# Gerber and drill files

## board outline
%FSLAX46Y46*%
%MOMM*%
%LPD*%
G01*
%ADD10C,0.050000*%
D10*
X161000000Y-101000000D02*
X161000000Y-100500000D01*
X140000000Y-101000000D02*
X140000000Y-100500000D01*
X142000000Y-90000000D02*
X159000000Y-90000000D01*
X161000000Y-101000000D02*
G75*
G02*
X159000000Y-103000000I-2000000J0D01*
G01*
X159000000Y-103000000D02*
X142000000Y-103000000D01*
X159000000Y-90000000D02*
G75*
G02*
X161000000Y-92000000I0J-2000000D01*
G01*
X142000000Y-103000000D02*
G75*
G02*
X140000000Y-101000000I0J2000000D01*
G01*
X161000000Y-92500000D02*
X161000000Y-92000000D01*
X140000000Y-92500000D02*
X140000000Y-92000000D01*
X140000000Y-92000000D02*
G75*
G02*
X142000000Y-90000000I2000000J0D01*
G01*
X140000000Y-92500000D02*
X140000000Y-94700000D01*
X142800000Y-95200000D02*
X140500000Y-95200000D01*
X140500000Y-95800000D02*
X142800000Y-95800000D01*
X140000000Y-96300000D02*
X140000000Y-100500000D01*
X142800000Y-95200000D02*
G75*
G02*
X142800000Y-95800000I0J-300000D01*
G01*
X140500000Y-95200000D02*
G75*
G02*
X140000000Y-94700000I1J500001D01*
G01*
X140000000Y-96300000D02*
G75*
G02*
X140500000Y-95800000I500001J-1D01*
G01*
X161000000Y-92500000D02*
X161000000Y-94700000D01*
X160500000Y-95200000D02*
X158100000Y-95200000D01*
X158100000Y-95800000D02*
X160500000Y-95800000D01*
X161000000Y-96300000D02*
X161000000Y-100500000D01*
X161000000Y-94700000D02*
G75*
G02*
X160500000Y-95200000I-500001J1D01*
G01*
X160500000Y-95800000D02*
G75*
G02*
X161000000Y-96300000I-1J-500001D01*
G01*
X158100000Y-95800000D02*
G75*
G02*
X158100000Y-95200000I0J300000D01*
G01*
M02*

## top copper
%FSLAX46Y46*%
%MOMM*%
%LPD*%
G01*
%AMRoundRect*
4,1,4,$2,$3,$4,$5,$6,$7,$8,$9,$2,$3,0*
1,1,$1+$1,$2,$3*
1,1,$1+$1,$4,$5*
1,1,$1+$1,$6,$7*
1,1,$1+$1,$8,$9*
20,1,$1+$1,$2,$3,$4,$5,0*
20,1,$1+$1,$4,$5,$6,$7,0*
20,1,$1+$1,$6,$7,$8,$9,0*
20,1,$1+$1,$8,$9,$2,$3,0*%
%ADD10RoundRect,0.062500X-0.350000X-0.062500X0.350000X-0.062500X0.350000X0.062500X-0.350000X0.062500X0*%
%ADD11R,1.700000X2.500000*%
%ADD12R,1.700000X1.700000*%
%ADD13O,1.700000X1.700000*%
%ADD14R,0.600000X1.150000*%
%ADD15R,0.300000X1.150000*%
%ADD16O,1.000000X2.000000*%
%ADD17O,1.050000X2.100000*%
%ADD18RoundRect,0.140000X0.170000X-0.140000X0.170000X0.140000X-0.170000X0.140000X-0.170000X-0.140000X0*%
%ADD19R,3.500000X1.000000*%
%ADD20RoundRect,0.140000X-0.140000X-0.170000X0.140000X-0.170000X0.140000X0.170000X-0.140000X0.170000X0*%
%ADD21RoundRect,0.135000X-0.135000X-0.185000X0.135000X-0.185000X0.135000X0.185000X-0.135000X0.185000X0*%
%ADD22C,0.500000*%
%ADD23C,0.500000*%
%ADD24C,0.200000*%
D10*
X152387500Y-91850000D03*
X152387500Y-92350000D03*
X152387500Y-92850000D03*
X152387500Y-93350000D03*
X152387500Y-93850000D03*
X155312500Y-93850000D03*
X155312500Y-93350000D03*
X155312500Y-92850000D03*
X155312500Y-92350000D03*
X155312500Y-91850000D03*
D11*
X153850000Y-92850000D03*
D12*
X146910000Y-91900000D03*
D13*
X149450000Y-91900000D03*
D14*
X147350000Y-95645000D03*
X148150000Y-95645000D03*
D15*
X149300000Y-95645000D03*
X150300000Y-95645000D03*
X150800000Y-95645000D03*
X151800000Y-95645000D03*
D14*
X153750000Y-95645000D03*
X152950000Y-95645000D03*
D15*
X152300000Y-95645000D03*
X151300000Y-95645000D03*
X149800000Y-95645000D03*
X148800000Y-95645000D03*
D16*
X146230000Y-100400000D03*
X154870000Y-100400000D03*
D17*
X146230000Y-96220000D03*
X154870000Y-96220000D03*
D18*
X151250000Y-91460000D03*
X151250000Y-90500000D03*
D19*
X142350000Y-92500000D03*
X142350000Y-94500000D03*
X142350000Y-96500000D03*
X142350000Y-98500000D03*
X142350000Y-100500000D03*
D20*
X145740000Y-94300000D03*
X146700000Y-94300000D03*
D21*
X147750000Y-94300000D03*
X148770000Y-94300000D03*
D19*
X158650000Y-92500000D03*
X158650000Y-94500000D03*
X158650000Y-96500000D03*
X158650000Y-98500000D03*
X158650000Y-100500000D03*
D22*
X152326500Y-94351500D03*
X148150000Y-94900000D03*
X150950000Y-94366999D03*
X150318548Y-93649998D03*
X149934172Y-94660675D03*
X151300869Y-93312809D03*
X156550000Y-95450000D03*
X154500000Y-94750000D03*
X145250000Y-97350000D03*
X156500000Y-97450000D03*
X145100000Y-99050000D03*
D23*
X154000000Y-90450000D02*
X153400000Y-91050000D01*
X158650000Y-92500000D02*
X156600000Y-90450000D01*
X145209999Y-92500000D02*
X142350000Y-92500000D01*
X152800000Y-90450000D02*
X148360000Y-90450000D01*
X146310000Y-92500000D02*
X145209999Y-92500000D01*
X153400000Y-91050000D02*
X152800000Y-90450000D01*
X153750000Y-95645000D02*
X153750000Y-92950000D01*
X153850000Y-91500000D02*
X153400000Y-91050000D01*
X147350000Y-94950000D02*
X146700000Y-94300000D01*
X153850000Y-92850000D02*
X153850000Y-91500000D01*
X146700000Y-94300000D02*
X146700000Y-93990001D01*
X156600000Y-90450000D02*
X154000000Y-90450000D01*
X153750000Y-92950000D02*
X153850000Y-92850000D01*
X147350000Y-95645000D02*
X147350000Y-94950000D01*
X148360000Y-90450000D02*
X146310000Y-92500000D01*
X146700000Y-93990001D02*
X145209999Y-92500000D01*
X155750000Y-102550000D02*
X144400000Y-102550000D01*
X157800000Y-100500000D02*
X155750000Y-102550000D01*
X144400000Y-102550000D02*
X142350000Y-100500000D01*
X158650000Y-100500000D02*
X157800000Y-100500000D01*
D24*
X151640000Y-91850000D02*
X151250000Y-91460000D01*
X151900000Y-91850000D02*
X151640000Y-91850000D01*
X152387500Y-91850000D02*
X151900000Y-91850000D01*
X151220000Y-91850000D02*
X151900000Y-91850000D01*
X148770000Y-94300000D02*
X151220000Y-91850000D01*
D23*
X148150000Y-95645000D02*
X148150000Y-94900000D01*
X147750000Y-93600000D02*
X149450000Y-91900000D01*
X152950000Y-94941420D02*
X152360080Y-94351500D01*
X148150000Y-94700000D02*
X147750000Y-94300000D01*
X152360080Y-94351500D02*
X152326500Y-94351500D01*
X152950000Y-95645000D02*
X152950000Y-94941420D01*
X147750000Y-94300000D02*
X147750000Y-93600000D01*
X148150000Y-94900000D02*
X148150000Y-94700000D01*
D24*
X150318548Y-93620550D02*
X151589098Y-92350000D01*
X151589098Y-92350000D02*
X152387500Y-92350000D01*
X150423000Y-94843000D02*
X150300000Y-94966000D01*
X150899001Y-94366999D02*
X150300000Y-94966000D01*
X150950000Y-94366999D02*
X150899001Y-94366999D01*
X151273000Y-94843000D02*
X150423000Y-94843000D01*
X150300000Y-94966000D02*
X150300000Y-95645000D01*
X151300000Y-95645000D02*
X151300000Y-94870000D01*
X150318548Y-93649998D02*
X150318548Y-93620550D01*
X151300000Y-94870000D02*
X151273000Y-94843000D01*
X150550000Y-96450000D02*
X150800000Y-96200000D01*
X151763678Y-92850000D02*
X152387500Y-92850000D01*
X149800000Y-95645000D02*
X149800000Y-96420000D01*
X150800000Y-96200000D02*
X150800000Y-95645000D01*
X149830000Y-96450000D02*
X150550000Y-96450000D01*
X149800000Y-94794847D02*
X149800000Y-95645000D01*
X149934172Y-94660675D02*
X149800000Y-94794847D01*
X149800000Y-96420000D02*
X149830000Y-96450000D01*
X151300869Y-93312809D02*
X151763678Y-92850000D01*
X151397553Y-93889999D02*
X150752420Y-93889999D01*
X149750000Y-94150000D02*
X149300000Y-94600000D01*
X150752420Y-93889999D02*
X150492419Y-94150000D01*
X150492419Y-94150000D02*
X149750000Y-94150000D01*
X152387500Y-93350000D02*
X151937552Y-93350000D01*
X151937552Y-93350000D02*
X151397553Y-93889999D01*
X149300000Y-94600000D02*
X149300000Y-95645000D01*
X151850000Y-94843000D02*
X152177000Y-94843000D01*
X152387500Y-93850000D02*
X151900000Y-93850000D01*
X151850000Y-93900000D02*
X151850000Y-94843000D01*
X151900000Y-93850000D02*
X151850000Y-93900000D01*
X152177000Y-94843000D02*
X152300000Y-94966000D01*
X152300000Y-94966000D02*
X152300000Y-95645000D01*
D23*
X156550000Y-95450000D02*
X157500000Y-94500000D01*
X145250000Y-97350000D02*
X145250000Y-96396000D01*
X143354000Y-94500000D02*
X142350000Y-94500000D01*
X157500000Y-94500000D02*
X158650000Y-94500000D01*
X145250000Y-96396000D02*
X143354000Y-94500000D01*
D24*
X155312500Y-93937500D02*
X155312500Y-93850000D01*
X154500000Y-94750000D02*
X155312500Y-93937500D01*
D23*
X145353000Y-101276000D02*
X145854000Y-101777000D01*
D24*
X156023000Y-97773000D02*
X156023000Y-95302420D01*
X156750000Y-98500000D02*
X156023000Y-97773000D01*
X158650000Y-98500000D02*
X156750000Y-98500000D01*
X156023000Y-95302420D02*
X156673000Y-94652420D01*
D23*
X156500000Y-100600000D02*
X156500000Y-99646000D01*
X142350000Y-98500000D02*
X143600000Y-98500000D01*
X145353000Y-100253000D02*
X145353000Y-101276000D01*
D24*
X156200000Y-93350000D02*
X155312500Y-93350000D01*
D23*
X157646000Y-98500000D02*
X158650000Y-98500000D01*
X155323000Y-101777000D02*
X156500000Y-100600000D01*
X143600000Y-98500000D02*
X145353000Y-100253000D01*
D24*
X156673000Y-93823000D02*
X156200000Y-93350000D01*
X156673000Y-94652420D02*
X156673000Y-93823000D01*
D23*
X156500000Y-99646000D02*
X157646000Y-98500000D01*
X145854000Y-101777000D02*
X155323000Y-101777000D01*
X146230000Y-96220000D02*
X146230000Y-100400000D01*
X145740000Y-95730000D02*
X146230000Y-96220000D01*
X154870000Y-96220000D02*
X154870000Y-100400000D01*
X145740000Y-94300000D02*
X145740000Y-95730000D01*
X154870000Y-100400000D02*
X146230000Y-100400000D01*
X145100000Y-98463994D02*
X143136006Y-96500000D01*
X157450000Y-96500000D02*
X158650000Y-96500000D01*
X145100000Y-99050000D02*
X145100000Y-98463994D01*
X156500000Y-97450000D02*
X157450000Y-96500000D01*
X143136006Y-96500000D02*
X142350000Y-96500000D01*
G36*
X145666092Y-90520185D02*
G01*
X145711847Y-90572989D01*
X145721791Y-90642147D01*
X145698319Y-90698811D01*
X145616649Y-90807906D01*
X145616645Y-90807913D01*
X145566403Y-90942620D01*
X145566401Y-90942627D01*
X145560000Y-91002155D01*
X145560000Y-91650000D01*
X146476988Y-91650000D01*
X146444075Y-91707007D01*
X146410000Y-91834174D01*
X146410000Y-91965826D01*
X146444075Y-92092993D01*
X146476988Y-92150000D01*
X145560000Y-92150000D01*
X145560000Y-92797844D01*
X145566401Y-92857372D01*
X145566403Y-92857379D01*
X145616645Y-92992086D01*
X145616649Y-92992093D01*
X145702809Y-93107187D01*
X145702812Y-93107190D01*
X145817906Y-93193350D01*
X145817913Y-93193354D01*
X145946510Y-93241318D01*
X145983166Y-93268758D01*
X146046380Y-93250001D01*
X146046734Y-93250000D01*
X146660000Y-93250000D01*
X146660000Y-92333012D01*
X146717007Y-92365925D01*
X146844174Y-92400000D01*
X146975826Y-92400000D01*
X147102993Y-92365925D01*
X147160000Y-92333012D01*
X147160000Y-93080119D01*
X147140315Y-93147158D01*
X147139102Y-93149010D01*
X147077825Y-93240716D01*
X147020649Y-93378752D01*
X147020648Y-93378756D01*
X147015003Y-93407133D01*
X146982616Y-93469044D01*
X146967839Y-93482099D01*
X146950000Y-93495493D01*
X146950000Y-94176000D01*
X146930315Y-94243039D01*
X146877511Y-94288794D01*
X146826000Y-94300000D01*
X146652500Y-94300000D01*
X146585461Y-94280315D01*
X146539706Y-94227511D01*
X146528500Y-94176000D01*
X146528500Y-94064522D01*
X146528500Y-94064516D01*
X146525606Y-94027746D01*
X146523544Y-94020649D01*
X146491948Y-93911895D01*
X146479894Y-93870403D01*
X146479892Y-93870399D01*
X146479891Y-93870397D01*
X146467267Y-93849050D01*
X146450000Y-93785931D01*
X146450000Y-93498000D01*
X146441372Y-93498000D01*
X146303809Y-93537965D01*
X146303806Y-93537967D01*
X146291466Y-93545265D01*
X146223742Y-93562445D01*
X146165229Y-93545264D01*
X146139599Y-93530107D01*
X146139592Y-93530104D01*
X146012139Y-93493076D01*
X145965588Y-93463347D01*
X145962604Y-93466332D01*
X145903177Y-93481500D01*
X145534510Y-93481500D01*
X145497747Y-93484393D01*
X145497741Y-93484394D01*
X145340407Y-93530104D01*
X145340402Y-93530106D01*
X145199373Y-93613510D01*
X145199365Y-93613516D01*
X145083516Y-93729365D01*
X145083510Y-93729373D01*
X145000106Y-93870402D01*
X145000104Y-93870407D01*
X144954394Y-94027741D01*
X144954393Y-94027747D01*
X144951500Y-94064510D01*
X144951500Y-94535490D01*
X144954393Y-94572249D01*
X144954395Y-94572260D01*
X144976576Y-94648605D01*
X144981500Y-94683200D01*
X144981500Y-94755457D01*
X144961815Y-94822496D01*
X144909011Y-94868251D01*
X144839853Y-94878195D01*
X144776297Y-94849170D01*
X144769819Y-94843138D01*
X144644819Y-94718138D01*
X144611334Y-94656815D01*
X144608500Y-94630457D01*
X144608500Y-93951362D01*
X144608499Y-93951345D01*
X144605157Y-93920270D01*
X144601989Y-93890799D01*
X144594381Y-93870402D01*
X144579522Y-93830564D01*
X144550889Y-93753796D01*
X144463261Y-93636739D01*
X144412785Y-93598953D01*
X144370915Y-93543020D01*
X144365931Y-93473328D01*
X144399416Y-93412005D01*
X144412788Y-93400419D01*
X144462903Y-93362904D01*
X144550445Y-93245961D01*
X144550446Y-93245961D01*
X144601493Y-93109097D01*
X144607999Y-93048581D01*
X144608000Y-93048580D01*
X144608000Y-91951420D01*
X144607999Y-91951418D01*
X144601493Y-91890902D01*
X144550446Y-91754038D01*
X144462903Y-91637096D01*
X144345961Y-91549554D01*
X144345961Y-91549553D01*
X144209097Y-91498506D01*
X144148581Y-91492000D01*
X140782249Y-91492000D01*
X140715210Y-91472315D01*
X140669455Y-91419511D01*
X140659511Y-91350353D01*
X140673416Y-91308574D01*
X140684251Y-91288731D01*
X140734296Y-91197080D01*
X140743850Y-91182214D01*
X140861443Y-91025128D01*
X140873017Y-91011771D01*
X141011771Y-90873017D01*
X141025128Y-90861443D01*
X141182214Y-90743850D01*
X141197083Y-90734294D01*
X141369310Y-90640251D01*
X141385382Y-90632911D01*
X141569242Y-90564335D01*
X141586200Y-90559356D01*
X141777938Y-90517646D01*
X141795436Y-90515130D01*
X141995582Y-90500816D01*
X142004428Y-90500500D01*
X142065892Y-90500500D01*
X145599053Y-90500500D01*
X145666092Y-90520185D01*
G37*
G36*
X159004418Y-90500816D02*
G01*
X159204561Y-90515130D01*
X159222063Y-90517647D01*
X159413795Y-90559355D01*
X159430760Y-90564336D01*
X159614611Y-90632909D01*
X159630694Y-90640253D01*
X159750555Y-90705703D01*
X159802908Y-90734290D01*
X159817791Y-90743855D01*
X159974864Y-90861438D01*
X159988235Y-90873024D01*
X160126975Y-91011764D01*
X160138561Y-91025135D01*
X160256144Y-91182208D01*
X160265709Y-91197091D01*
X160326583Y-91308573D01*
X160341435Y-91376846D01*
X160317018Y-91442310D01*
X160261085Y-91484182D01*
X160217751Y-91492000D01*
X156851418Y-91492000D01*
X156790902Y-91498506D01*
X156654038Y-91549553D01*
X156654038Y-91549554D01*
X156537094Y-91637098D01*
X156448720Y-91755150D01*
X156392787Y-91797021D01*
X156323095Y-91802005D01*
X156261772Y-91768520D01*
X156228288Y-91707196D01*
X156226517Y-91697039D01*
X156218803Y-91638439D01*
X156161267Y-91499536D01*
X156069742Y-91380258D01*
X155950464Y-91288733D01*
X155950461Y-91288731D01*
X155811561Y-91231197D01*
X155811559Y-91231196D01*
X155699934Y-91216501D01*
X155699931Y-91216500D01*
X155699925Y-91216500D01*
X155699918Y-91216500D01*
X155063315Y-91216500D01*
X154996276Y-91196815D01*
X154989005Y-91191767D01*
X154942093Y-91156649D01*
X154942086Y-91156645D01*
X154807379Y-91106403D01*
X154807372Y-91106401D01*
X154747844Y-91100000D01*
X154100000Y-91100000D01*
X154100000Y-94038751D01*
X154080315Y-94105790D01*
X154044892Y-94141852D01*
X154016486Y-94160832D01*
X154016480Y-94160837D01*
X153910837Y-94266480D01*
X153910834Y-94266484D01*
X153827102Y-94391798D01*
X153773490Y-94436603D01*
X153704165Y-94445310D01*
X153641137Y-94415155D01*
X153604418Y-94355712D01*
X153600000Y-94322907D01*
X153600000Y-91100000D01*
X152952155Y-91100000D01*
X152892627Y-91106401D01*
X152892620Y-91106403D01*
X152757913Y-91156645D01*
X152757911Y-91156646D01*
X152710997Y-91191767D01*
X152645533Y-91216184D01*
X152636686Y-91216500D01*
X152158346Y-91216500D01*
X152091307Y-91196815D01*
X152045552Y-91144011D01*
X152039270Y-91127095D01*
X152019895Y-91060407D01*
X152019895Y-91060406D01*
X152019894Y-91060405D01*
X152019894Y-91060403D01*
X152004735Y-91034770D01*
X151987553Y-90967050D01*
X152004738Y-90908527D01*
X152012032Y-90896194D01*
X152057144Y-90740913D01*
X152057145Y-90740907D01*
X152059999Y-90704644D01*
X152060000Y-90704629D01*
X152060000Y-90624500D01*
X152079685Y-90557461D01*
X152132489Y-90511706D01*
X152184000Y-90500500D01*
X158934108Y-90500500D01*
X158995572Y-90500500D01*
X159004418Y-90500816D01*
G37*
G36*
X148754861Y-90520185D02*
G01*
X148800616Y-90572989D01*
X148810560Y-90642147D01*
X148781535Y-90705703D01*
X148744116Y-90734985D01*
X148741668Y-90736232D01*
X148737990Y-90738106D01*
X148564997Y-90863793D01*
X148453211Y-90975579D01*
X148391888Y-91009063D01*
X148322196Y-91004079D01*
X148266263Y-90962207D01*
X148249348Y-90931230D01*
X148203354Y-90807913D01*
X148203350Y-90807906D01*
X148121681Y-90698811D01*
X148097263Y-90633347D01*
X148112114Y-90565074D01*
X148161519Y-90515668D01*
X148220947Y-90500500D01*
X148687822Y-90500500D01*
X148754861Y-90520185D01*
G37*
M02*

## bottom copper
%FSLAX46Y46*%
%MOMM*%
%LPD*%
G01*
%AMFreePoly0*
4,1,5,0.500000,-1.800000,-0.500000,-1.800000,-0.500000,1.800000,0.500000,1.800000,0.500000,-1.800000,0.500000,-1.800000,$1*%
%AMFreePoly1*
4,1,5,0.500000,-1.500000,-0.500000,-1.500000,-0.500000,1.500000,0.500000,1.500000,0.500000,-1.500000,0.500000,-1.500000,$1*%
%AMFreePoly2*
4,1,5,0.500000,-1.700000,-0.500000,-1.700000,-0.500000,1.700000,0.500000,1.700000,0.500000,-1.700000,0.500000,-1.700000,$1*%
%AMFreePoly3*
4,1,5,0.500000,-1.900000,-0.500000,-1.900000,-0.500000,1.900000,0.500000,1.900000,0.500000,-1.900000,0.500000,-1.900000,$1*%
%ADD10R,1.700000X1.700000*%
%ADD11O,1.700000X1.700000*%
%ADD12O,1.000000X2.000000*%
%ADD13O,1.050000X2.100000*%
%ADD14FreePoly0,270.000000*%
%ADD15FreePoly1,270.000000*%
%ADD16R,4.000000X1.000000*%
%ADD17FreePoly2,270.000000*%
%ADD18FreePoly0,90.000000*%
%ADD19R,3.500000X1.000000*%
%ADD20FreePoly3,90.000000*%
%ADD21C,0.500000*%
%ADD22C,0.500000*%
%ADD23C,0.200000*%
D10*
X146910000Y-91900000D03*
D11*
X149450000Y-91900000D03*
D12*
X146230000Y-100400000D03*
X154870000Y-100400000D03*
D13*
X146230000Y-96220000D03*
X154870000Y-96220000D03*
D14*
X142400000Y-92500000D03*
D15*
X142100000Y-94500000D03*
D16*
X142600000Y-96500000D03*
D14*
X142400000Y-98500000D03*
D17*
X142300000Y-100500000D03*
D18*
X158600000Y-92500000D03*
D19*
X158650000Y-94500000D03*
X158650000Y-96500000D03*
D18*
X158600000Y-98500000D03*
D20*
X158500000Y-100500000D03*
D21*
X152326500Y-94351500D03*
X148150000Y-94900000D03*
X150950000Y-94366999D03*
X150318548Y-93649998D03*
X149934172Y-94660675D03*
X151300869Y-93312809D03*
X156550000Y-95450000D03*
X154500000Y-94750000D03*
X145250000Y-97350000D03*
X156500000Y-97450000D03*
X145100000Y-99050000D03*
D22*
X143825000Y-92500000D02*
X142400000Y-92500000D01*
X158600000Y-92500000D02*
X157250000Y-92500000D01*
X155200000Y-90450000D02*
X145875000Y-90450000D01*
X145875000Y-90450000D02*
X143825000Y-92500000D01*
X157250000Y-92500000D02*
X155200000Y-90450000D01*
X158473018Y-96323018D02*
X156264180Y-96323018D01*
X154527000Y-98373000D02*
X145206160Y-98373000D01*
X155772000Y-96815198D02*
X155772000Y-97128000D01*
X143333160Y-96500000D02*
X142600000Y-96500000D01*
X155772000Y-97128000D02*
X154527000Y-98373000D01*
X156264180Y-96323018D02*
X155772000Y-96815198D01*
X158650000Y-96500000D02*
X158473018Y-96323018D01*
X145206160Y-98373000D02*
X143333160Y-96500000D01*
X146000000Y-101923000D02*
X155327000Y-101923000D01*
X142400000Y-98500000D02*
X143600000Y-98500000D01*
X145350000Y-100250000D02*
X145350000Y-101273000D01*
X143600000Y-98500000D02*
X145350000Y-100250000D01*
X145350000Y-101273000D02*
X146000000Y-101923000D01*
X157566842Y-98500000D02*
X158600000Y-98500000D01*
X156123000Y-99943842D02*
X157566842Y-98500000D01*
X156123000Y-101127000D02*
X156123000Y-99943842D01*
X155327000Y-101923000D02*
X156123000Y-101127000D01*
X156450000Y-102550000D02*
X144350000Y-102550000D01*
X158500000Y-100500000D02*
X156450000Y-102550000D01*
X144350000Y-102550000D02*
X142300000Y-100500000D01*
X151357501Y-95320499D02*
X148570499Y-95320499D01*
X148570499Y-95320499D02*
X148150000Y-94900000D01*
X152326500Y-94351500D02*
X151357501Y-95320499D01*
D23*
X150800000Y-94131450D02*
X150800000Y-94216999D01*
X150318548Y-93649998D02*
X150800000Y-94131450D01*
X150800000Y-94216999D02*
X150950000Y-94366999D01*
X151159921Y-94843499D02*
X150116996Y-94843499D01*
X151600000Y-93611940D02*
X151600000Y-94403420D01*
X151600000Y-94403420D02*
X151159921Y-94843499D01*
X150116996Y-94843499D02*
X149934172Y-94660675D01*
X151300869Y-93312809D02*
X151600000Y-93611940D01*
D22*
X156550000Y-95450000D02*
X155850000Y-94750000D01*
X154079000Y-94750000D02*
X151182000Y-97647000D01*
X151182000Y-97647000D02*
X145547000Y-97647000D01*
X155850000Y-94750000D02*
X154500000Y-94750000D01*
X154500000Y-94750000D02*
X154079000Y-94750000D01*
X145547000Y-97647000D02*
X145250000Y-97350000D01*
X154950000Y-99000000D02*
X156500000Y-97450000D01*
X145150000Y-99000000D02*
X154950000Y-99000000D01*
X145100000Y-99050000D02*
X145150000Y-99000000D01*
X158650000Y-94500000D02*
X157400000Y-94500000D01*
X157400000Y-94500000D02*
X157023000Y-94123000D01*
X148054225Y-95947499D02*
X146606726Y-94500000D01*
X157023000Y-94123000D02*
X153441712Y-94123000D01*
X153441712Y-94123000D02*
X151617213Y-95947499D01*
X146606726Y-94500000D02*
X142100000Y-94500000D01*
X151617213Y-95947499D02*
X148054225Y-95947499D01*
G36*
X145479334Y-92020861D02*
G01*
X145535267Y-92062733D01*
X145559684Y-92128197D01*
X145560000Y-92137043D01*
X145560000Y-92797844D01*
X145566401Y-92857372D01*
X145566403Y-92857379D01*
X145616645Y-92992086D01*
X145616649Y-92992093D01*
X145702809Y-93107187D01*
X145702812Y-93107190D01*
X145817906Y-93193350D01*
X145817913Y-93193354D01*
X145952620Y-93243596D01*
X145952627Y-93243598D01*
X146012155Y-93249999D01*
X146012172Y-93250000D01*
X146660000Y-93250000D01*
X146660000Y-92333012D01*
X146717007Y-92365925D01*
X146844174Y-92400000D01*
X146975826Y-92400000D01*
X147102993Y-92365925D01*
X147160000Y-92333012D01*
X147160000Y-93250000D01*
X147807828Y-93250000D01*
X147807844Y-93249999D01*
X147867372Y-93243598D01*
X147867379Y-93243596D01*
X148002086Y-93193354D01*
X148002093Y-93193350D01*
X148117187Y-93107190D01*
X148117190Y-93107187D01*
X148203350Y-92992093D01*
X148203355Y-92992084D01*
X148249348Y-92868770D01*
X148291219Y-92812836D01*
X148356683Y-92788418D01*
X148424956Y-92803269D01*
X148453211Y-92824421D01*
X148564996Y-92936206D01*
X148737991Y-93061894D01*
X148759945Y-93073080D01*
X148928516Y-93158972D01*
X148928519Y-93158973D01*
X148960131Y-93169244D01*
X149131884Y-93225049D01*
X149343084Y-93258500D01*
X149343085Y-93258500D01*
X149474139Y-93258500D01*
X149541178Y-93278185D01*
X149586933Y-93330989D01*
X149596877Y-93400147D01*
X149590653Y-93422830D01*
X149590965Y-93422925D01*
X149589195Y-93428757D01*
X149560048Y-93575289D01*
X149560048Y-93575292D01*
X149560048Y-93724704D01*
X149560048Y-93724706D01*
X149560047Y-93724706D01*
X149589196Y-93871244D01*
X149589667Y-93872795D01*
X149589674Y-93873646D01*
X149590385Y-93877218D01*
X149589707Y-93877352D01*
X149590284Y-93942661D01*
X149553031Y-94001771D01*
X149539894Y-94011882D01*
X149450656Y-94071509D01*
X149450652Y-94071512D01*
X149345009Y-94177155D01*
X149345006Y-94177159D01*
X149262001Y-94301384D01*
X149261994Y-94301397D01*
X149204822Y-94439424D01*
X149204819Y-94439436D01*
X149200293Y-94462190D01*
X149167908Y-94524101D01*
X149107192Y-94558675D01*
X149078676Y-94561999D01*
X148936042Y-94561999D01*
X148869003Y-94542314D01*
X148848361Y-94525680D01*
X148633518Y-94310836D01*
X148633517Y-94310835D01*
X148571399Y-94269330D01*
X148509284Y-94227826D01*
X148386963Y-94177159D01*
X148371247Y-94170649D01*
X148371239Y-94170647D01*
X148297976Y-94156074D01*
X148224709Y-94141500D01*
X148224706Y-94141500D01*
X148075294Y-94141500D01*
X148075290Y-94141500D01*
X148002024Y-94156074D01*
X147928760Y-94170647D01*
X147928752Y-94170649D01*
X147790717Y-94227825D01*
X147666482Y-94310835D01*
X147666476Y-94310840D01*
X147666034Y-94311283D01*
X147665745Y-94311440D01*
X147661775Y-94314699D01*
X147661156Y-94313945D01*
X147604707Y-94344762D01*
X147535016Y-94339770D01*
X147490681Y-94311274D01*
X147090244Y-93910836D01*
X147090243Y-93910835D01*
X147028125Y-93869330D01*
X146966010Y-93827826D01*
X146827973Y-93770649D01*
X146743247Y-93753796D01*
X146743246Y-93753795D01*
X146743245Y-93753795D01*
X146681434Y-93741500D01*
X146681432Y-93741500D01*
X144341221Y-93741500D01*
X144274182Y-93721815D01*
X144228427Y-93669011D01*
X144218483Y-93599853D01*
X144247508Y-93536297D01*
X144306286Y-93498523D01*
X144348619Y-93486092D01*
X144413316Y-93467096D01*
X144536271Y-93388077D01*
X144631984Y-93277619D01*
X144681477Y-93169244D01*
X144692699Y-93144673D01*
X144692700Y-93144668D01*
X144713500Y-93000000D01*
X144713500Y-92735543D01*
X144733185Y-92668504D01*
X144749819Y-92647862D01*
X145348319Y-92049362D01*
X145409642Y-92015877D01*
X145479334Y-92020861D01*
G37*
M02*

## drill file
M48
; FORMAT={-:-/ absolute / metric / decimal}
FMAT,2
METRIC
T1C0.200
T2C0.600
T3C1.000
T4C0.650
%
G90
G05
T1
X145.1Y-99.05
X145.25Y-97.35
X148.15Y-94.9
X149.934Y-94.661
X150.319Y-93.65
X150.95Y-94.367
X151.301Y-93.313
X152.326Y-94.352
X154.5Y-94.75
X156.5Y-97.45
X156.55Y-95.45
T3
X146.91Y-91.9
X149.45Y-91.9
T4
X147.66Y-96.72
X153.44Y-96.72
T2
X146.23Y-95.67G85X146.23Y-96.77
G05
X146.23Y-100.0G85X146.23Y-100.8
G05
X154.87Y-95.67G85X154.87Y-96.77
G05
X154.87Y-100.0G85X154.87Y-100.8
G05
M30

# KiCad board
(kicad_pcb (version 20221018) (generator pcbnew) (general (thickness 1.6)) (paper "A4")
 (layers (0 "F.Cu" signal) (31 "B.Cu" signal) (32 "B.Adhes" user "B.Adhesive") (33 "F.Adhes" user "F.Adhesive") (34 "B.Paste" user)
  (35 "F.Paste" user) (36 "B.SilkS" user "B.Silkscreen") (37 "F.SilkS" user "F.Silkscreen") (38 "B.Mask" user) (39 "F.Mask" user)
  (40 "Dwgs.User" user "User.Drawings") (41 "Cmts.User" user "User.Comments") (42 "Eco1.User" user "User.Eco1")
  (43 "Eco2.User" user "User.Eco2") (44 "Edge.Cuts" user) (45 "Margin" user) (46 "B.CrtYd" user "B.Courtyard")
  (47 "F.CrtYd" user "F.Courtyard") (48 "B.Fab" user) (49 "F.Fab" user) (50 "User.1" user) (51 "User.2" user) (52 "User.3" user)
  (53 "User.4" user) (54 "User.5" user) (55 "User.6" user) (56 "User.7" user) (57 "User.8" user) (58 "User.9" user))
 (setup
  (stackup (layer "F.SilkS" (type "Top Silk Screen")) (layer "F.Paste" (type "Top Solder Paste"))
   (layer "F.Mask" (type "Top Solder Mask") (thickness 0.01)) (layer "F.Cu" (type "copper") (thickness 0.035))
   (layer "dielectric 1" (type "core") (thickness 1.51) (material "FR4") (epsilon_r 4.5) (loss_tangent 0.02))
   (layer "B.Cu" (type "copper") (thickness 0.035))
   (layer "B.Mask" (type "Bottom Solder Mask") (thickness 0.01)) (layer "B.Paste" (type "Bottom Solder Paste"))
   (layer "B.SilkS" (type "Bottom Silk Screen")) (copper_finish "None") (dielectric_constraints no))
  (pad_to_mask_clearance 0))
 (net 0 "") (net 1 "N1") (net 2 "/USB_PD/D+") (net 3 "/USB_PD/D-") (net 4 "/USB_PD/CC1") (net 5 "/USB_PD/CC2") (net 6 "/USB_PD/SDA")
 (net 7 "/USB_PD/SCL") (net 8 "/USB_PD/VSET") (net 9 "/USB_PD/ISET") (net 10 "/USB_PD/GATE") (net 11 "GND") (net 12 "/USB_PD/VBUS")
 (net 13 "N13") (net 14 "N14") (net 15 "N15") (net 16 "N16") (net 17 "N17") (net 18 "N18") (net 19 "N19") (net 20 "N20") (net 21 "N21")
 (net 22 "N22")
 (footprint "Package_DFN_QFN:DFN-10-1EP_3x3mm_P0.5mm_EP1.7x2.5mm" (layer "F.Cu") (at 153.85 92.85)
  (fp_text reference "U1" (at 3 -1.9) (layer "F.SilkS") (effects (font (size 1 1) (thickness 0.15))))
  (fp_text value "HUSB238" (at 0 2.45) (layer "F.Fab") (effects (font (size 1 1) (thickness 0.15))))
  (pad "" smd roundrect (at -0.425 -0.625) (size 0.69 1.01) (layers "F.Paste") (roundrect_rratio 0.25))
  (pad "" smd roundrect (at -0.425 0.625) (size 0.69 1.01) (layers "F.Paste") (roundrect_rratio 0.25))
  (pad "" smd roundrect (at 0.425 -0.625) (size 0.69 1.01) (layers "F.Paste") (roundrect_rratio 0.25))
  (pad "" smd roundrect (at 0.425 0.625) (size 0.69 1.01) (layers "F.Paste") (roundrect_rratio 0.25))
  (pad "1" smd roundrect (at -1.4625 -1) (size 0.825 0.25) (layers "F.Cu" "F.Paste" "F.Mask") (roundrect_rratio 0.25) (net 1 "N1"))
  (pad "2" smd roundrect (at -1.4625 -0.5) (size 0.825 0.25) (layers "F.Cu" "F.Paste" "F.Mask") (roundrect_rratio 0.25) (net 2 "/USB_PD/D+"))
  (pad "3" smd roundrect (at -1.4625 0) (size 0.825 0.25) (layers "F.Cu" "F.Paste" "F.Mask") (roundrect_rratio 0.25) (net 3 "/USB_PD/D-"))
  (pad "4" smd roundrect (at -1.4625 0.5) (size 0.825 0.25) (layers "F.Cu" "F.Paste" "F.Mask") (roundrect_rratio 0.25) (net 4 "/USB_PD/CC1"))
  (pad "5" smd roundrect (at -1.4625 1) (size 0.825 0.25) (layers "F.Cu" "F.Paste" "F.Mask") (roundrect_rratio 0.25) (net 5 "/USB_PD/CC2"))
  (pad "6" smd roundrect (at 1.4625 1) (size 0.825 0.25) (layers "F.Cu" "F.Paste" "F.Mask") (roundrect_rratio 0.25) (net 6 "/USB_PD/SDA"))
  (pad "7" smd roundrect (at 1.4625 0.5) (size 0.825 0.25) (layers "F.Cu" "F.Paste" "F.Mask") (roundrect_rratio 0.25) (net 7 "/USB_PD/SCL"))
  (pad "8" smd roundrect (at 1.4625 0) (size 0.825 0.25) (layers "F.Cu" "F.Paste" "F.Mask") (roundrect_rratio 0.25) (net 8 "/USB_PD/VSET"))
  (pad "9" smd roundrect (at 1.4625 -0.5) (size 0.825 0.25) (layers "F.Cu" "F.Paste" "F.Mask") (roundrect_rratio 0.25)
   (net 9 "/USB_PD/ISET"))
  (pad "10" smd roundrect (at 1.4625 -1) (size 0.825 0.25) (layers "F.Cu" "F.Paste" "F.Mask") (roundrect_rratio 0.25)
   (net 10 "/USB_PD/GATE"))
  (pad "11" smd rect (at 0 0) (size 1.7 2.5) (layers "F.Cu" "F.Mask") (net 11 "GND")))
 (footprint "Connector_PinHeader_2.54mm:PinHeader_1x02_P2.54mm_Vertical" (layer "F.Cu") (at 146.91 91.9 90)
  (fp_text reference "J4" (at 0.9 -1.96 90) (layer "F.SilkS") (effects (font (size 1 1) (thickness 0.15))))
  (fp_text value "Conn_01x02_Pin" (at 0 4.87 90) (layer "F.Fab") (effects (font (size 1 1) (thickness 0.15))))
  (pad "1" thru_hole rect (at 0 0 90) (size 1.7 1.7) (drill 1) (layers "*.Cu" "*.Mask") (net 11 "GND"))
  (pad "2" thru_hole oval (at 0 2.54 90) (size 1.7 1.7) (drill 1) (layers "*.Cu" "*.Mask") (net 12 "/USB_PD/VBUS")))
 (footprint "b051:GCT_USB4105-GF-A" (layer "F.Cu") (at 150.55 100.4)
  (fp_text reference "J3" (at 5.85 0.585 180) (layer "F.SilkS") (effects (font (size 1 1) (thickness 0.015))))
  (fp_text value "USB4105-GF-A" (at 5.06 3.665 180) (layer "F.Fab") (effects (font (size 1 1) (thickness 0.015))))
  (pad "" np_thru_hole circle (at -2.89 -3.68) (size 0.65 0.65) (drill 0.65) (layers "*.Cu" "*.Mask"))
  (pad "" np_thru_hole circle (at 2.89 -3.68) (size 0.65 0.65) (drill 0.65) (layers "*.Cu" "*.Mask"))
  (pad "A1/B12" smd rect (at -3.2 -4.755) (size 0.6 1.15) (layers "F.Cu" "F.Paste" "F.Mask") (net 11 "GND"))
  (pad "A4/B9" smd rect (at -2.4 -4.755) (size 0.6 1.15) (layers "F.Cu" "F.Paste" "F.Mask") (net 12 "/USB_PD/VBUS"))
  (pad "A5" smd rect (at -1.25 -4.755) (size 0.3 1.15) (layers "F.Cu" "F.Paste" "F.Mask") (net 4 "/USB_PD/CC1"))
  (pad "A6" smd rect (at -0.25 -4.755) (size 0.3 1.15) (layers "F.Cu" "F.Paste" "F.Mask") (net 2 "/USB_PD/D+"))
  (pad "A7" smd rect (at 0.25 -4.755) (size 0.3 1.15) (layers "F.Cu" "F.Paste" "F.Mask") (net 3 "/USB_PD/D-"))
  (pad "A8" smd rect (at 1.25 -4.755) (size 0.3 1.15) (layers "F.Cu" "F.Paste" "F.Mask") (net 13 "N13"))
  (pad "B1/A12" smd rect (at 3.2 -4.755) (size 0.6 1.15) (layers "F.Cu" "F.Paste" "F.Mask") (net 11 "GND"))
  (pad "B4/A9" smd rect (at 2.4 -4.755) (size 0.6 1.15) (layers "F.Cu" "F.Paste" "F.Mask") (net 12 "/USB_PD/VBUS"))
  (pad "B5" smd rect (at 1.75 -4.755) (size 0.3 1.15) (layers "F.Cu" "F.Paste" "F.Mask") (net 5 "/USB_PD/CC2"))
  (pad "B6" smd rect (at 0.75 -4.755) (size 0.3 1.15) (layers "F.Cu" "F.Paste" "F.Mask") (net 2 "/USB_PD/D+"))
  (pad "B7" smd rect (at -0.75 -4.755) (size 0.3 1.15) (layers "F.Cu" "F.Paste" "F.Mask") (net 3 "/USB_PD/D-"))
  (pad "B8" smd rect (at -1.75 -4.755) (size 0.3 1.15) (layers "F.Cu" "F.Paste" "F.Mask") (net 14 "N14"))
  (pad "G1" thru_hole oval (at -4.32 0) (size 1 2) (drill oval 0.6 1.4) (layers "*.Cu" "*.Mask") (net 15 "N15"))
  (pad "G2" thru_hole oval (at 4.32 0) (size 1 2) (drill oval 0.6 1.4) (layers "*.Cu" "*.Mask") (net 15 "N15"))
  (pad "G3" thru_hole oval (at -4.32 -4.18) (size 1.05 2.1) (drill oval 0.6 1.7) (layers "*.Cu" "*.Mask") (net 15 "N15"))
  (pad "G4" thru_hole oval (at 4.32 -4.18) (size 1.05 2.1) (drill oval 0.6 1.7) (layers "*.Cu" "*.Mask") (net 15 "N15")))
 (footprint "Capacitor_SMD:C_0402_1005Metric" (layer "F.Cu") (at 151.25 90.98 90)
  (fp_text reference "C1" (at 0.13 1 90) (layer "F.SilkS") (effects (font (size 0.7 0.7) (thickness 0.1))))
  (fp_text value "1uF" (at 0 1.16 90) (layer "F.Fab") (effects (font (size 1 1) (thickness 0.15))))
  (pad "1" smd roundrect (at -0.48 0 90) (size 0.56 0.62) (layers "F.Cu" "F.Paste" "F.Mask") (roundrect_rratio 0.25) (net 1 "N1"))
  (pad "2" smd roundrect (at 0.48 0 90) (size 0.56 0.62) (layers "F.Cu" "F.Paste" "F.Mask") (roundrect_rratio 0.25) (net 11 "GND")))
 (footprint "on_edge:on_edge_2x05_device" (layer "F.Cu") (at 140 96.5 -90)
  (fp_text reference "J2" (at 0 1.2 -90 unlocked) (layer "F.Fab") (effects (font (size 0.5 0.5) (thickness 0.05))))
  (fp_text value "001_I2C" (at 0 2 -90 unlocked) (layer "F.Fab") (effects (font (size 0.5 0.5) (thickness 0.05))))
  (fp_line (start -4 0) (end -1.8 0) (stroke (width 0.05) (type solid)) (layer "Edge.Cuts"))
  (fp_line (start -1.3 -2.8) (end -1.3 -0.5) (stroke (width 0.05) (type solid)) (layer "Edge.Cuts"))
  (fp_line (start -0.7 -0.5) (end -0.7 -2.8) (stroke (width 0.05) (type solid)) (layer "Edge.Cuts"))
  (fp_line (start -0.2 0) (end 4 0) (stroke (width 0.05) (type solid)) (layer "Edge.Cuts"))
  (fp_arc (start -1.3 -2.8) (mid -1 -3.1) (end -0.7 -2.8) (stroke (width 0.05) (type solid)) (layer "Edge.Cuts"))
  (fp_arc (start -1.3 -0.5) (mid -1.446447 -0.146447) (end -1.8 0) (stroke (width 0.05) (type solid)) (layer "Edge.Cuts"))
  (fp_arc (start -0.2 0) (mid -0.553553 -0.146447) (end -0.7 -0.5) (stroke (width 0.05) (type solid)) (layer "Edge.Cuts"))
  (pad "1" smd rect (at -4 -2.35 90) (size 1 3.5) (layers "F.Cu" "F.Mask") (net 11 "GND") (zone_connect 0))
  (pad "2" smd rect (at -2 -2.35 270) (size 1 3.5) (layers "F.Cu" "F.Mask") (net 6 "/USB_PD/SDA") (zone_connect 0))
  (pad "3" smd rect (at 0 -2.35 270) (size 1 3.5) (layers "F.Cu" "F.Mask") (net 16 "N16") (zone_connect 0))
  (pad "4" smd rect (at 2 -2.35 90) (size 1 3.5) (layers "F.Cu" "F.Mask") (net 7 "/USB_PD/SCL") (zone_connect 0))
  (pad "5" smd rect (at 4 -2.35 90) (size 1 3.5) (layers "F.Cu" "F.Mask") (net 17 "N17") (zone_connect 0))
  (pad "6" smd custom (at -4 -2.4 270) (size 1 3.6) (layers "B.Cu" "B.Mask") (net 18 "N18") (zone_connect 0)
   (options (clearance outline) (anchor rect)) (primitives))
  (pad "7" smd custom (at -2 -2.1 270) (size 1 3) (layers "B.Cu" "B.Mask") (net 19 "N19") (zone_connect 0)
   (options (clearance outline) (anchor rect)) (primitives))
  (pad "8" smd rect (at 0 -2.6 270) (size 1 4) (layers "B.Cu" "B.Mask") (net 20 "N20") (zone_connect 0))
  (pad "9" smd custom (at 2 -2.4 270) (size 1 3.6) (layers "B.Cu" "B.Mask") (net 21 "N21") (zone_connect 0)
   (options (clearance outline) (anchor rect)) (primitives))
  (pad "10" smd custom (at 4 -2.3 270) (size 1 3.4) (layers "B.Cu" "B.Mask") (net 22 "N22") (zone_connect 0)
   (options (clearance outline) (anchor rect)) (primitives))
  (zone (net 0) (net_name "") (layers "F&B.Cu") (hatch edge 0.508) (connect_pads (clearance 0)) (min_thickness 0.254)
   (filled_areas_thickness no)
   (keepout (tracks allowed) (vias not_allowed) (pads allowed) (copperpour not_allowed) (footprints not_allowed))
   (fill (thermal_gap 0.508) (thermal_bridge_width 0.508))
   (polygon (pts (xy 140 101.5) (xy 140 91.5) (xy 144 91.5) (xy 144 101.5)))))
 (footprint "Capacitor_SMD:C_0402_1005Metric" (layer "F.Cu") (at 146.22 94.3)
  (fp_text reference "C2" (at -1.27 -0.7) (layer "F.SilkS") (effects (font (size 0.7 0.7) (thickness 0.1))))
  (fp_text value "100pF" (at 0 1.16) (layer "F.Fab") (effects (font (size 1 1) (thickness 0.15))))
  (pad "1" smd roundrect (at -0.48 0) (size 0.56 0.62) (layers "F.Cu" "F.Paste" "F.Mask") (roundrect_rratio 0.25) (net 15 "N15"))
  (pad "2" smd roundrect (at 0.48 0) (size 0.56 0.62) (layers "F.Cu" "F.Paste" "F.Mask") (roundrect_rratio 0.25) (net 11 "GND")))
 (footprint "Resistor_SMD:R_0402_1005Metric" (layer "F.Cu") (at 148.26 94.3)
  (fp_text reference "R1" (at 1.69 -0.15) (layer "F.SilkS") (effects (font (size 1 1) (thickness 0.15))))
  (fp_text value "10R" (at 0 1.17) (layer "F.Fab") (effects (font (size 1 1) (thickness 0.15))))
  (pad "1" smd roundrect (at -0.51 0) (size 0.54 0.64) (layers "F.Cu" "F.Paste" "F.Mask") (roundrect_rratio 0.25) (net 12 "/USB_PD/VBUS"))
  (pad "2" smd roundrect (at 0.51 0) (size 0.54 0.64) (layers "F.Cu" "F.Paste" "F.Mask") (roundrect_rratio 0.25) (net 1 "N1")))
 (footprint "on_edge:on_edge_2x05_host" (layer "F.Cu") (at 161 96.5 -90)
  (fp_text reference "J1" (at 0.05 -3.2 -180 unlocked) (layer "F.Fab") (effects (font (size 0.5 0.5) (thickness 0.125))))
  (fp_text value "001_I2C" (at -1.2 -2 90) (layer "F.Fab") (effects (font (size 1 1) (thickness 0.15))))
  (fp_line (start -4 0) (end -1.8 0) (stroke (width 0.05) (type solid)) (layer "Edge.Cuts"))
  (fp_line (start -1.3 0.5) (end -1.3 2.9) (stroke (width 0.05) (type solid)) (layer "Edge.Cuts"))
  (fp_line (start -0.7 2.9) (end -0.7 0.5) (stroke (width 0.05) (type solid)) (layer "Edge.Cuts"))
  (fp_line (start -0.2 0) (end 4 0) (stroke (width 0.05) (type solid)) (layer "Edge.Cuts"))
  (fp_arc (start -1.8 0) (mid -1.446447 0.146447) (end -1.3 0.5) (stroke (width 0.05) (type solid)) (layer "Edge.Cuts"))
  (fp_arc (start -0.7 0.5) (mid -0.553553 0.146447) (end -0.2 0) (stroke (width 0.05) (type solid)) (layer "Edge.Cuts"))
  (fp_arc (start -0.7 2.9) (mid -1 3.2) (end -1.3 2.9) (stroke (width 0.05) (type solid)) (layer "Edge.Cuts"))
  (pad "1" smd rect (at -4 2.35 270) (size 1 3.5) (layers "F.Cu" "F.Mask") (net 11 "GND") (zone_connect 0))
  (pad "2" smd rect (at -2 2.35 270) (size 1 3.5) (layers "F.Cu" "F.Mask") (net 6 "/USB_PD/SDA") (zone_connect 0))
  (pad "3" smd rect (at 0 2.35 270) (size 1 3.5) (layers "F.Cu" "F.Mask") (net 16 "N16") (zone_connect 0))
  (pad "4" smd rect (at 2 2.35 270) (size 1 3.5) (layers "F.Cu" "F.Mask") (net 7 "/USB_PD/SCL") (zone_connect 0))
  (pad "5" smd rect (at 4 2.35 270) (size 1 3.5) (layers "F.Cu" "F.Mask") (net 17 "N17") (zone_connect 0))
  (pad "6" smd custom (at -4 2.4 90) (size 1 3.6) (layers "B.Cu" "B.Mask") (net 18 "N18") (zone_connect 0)
   (options (clearance outline) (anchor rect)) (primitives))
  (pad "7" smd rect (at -2 2.35 90) (size 1 3.5) (layers "B.Cu" "B.Mask") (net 19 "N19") (zone_connect 0))
  (pad "8" smd rect (at 0 2.35 90) (size 1 3.5) (layers "B.Cu" "B.Mask") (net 20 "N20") (zone_connect 0))
  (pad "9" smd custom (at 2 2.4 90) (size 1 3.6) (layers "B.Cu" "B.Mask") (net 21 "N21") (zone_connect 0)
   (options (clearance outline) (anchor rect)) (primitives))
  (pad "10" smd custom (at 4 2.5 90) (size 1 3.8) (layers "B.Cu" "B.Mask") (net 22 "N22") (zone_connect 0)
   (options (clearance outline) (anchor rect)) (primitives))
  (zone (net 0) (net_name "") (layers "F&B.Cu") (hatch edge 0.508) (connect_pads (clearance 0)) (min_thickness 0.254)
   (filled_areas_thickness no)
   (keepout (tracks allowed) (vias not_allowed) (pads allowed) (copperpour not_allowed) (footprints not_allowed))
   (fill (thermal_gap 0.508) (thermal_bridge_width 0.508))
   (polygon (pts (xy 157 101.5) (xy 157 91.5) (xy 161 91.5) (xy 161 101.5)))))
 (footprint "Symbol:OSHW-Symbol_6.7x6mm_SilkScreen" (layer "B.Cu") (at 150.6 97.6 180)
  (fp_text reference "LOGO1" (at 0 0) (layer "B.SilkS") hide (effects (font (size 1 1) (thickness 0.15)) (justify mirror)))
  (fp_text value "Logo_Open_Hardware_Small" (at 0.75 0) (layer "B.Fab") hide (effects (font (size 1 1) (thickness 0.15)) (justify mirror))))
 (gr_line (start 161 101) (end 161 100.5) (stroke (width 0.05) (type solid)) (layer "Edge.Cuts"))
 (gr_line (start 140 101) (end 140 100.5) (stroke (width 0.05) (type solid)) (layer "Edge.Cuts"))
 (gr_line (start 142 90) (end 159 90) (stroke (width 0.05) (type solid)) (layer "Edge.Cuts"))
 (gr_arc (start 161 101) (mid 160.414214 102.414214) (end 159 103) (stroke (width 0.05) (type solid)) (layer "Edge.Cuts"))
 (gr_line (start 159 103) (end 142 103) (stroke (width 0.05) (type solid)) (layer "Edge.Cuts"))
 (gr_arc (start 159 90) (mid 160.414214 90.585786) (end 161 92) (stroke (width 0.05) (type solid)) (layer "Edge.Cuts"))
 (gr_arc (start 142 103) (mid 140.585786 102.414214) (end 140 101) (stroke (width 0.05) (type solid)) (layer "Edge.Cuts"))
 (gr_line (start 161 92.5) (end 161 92) (stroke (width 0.05) (type solid)) (layer "Edge.Cuts"))
 (gr_line (start 140 92.5) (end 140 92) (stroke (width 0.05) (type solid)) (layer "Edge.Cuts"))
 (gr_arc (start 140 92) (mid 140.585786 90.585786) (end 142 90) (stroke (width 0.05) (type solid)) (layer "Edge.Cuts"))
 (segment (start 154 90.45) (end 153.4 91.05) (width 0.5) (layer "F.Cu") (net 11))
 (segment (start 158.65 92.5) (end 156.6 90.45) (width 0.5) (layer "F.Cu") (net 11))
 (segment (start 145.209999 92.5) (end 142.35 92.5) (width 0.5) (layer "F.Cu") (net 11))
 (segment (start 152.8 90.45) (end 148.36 90.45) (width 0.5) (layer "F.Cu") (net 11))
 (segment (start 146.31 92.5) (end 145.209999 92.5) (width 0.5) (layer "F.Cu") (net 11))
 (segment (start 153.4 91.05) (end 152.8 90.45) (width 0.5) (layer "F.Cu") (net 11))
 (segment (start 153.75 95.645) (end 153.75 92.95) (width 0.5) (layer "F.Cu") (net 11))
 (segment (start 153.85 91.5) (end 153.4 91.05) (width 0.5) (layer "F.Cu") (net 11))
 (segment (start 147.35 94.95) (end 146.7 94.3) (width 0.5) (layer "F.Cu") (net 11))
 (segment (start 153.85 92.85) (end 153.85 91.5) (width 0.5) (layer "F.Cu") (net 11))
 (segment (start 146.7 94.3) (end 146.7 93.990001) (width 0.5) (layer "F.Cu") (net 11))
 (segment (start 156.6 90.45) (end 154 90.45) (width 0.5) (layer "F.Cu") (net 11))
 (segment (start 153.75 92.95) (end 153.85 92.85) (width 0.5) (layer "F.Cu") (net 11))
 (segment (start 147.35 95.645) (end 147.35 94.95) (width 0.5) (layer "F.Cu") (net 11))
 (segment (start 148.36 90.45) (end 146.31 92.5) (width 0.5) (layer "F.Cu") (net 11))
 (segment (start 146.7 93.990001) (end 145.209999 92.5) (width 0.5) (layer "F.Cu") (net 11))
 (segment (start 143.825 92.5) (end 142.4 92.5) (width 0.5) (layer "B.Cu") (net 18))
 (segment (start 158.6 92.5) (end 157.25 92.5) (width 0.5) (layer "B.Cu") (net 18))
 (segment (start 155.2 90.45) (end 145.875 90.45) (width 0.5) (layer "B.Cu") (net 18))
 (segment (start 145.875 90.45) (end 143.825 92.5) (width 0.5) (layer "B.Cu") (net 18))
 (segment (start 157.25 92.5) (end 155.2 90.45) (width 0.5) (layer "B.Cu") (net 18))
 (segment (start 155.75 102.55) (end 144.4 102.55) (width 0.5) (layer "F.Cu") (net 17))
 (segment (start 157.8 100.5) (end 155.75 102.55) (width 0.5) (layer "F.Cu") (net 17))
 (segment (start 144.4 102.55) (end 142.35 100.5) (width 0.5) (layer "F.Cu") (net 17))
 (segment (start 158.65 100.5) (end 157.8 100.5) (width 0.5) (layer "F.Cu") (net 17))
 (segment (start 158.473018 96.323018) (end 156.26418 96.323018) (width 0.5) (layer "B.Cu") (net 20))
 (segment (start 154.527 98.373) (end 145.20616 98.373) (width 0.5) (layer "B.Cu") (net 20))
 (segment (start 155.772 96.815198) (end 155.772 97.128) (width 0.5) (layer "B.Cu") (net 20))
 (segment (start 143.33316 96.5) (end 142.6 96.5) (width 0.5) (layer "B.Cu") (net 20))
 (segment (start 155.772 97.128) (end 154.527 98.373) (width 0.5) (layer "B.Cu") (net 20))
 (segment (start 156.26418 96.323018) (end 155.772 96.815198) (width 0.5) (layer "B.Cu") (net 20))
 (segment (start 158.65 96.5) (end 158.473018 96.323018) (width 0.5) (layer "B.Cu") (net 20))
 (segment (start 145.20616 98.373) (end 143.33316 96.5) (width 0.5) (layer "B.Cu") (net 20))
 (segment (start 146 101.923) (end 155.327 101.923) (width 0.5) (layer "B.Cu") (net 21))
 (segment (start 142.4 98.5) (end 143.6 98.5) (width 0.5) (layer "B.Cu") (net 21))
 (segment (start 145.35 100.25) (end 145.35 101.273) (width 0.5) (layer "B.Cu") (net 21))
 (segment (start 143.6 98.5) (end 145.35 100.25) (width 0.5) (layer "B.Cu") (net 21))
 (segment (start 145.35 101.273) (end 146 101.923) (width 0.5) (layer "B.Cu") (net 21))
 (segment (start 157.566842 98.5) (end 158.6 98.5) (width 0.5) (layer "B.Cu") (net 21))
 (segment (start 156.123 99.943842) (end 157.566842 98.5) (width 0.5) (layer "B.Cu") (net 21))
 (segment (start 156.123 101.127) (end 156.123 99.943842) (width 0.5) (layer "B.Cu") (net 21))
 (segment (start 155.327 101.923) (end 156.123 101.127) (width 0.5) (layer "B.Cu") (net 21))
 (segment (start 156.45 102.55) (end 144.35 102.55) (width 0.5) (layer "B.Cu") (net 22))
 (segment (start 158.5 100.5) (end 156.45 102.55) (width 0.5) (layer "B.Cu") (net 22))
 (segment (start 144.35 102.55) (end 142.3 100.5) (width 0.5) (layer "B.Cu") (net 22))
 (segment (start 151.64 91.85) (end 151.25 91.46) (width 0.2) (layer "F.Cu") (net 1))
 (segment (start 151.9 91.85) (end 151.64 91.85) (width 0.2) (layer "F.Cu") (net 1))
 (segment (start 152.3875 91.85) (end 151.9 91.85) (width 0.2) (layer "F.Cu") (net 1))
 (segment (start 151.22 91.85) (end 151.9 91.85) (width 0.2) (layer "F.Cu") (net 1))
 (segment (start 148.77 94.3) (end 151.22 91.85) (width 0.2) (layer "F.Cu") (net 1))
 (segment (start 148.15 95.645) (end 148.15 94.9) (width 0.5) (layer "F.Cu") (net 12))
 (segment (start 147.75 93.6) (end 149.45 91.9) (width 0.5) (layer "F.Cu") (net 12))
 (segment (start 152.95 94.94142) (end 152.36008 94.3515) (width 0.5) (layer "F.Cu") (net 12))
 (segment (start 148.15 94.7) (end 147.75 94.3) (width 0.5) (layer "F.Cu") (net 12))
 (segment (start 152.36008 94.3515) (end 152.3265 94.3515) (width 0.5) (layer "F.Cu") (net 12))
 (segment (start 152.95 95.645) (end 152.95 94.94142) (width 0.5) (layer "F.Cu") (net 12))
 (segment (start 147.75 94.3) (end 147.75 93.6) (width 0.5) (layer "F.Cu") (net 12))
 (segment (start 148.15 94.9) (end 148.15 94.7) (width 0.5) (layer "F.Cu") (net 12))
 (via (at 152.3265 94.3515) (size 0.5) (drill 0.2) (layers "F.Cu" "B.Cu") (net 12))
 (via (at 148.15 94.9) (size 0.5) (drill 0.2) (layers "F.Cu" "B.Cu") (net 12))
 (segment (start 151.357501 95.320499) (end 148.570499 95.320499) (width 0.5) (layer "B.Cu") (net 12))
 (segment (start 148.570499 95.320499) (end 148.15 94.9) (width 0.5) (layer "B.Cu") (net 12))
 (segment (start 152.3265 94.3515) (end 151.357501 95.320499) (width 0.5) (layer "B.Cu") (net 12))
 (segment (start 150.318548 93.62055) (end 151.589098 92.35) (width 0.2) (layer "F.Cu") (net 2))
 (segment (start 151.589098 92.35) (end 152.3875 92.35) (width 0.2) (layer "F.Cu") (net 2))
 (segment (start 150.423 94.843) (end 150.3 94.966) (width 0.2) (layer "F.Cu") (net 2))
 (segment (start 150.899001 94.366999) (end 150.3 94.966) (width 0.2) (layer "F.Cu") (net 2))
 (segment (start 150.95 94.366999) (end 150.899001 94.366999) (width 0.2) (layer "F.Cu") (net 2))
 (segment (start 151.273 94.843) (end 150.423 94.843) (width 0.2) (layer "F.Cu") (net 2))
 (segment (start 150.3 94.966) (end 150.3 95.645) (width 0.2) (layer "F.Cu") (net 2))
 (segment (start 151.3 95.645) (end 151.3 94.87) (width 0.2) (layer "F.Cu") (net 2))
 (segment (start 150.318548 93.649998) (end 150.318548 93.62055) (width 0.2) (layer "F.Cu") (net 2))
 (segment (start 151.3 94.87) (end 151.273 94.843) (width 0.2) (layer "F.Cu") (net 2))
 (via (at 150.95 94.366999) (size 0.5) (drill 0.2) (layers "F.Cu" "B.Cu") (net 2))
 (via (at 150.318548 93.649998) (size 0.5) (drill 0.2) (layers "F.Cu" "B.Cu") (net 2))
 (segment (start 150.8 94.13145) (end 150.8 94.216999) (width 0.2) (layer "B.Cu") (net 2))
 (segment (start 150.318548 93.649998) (end 150.8 94.13145) (width 0.2) (layer "B.Cu") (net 2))
 (segment (start 150.8 94.216999) (end 150.95 94.366999) (width 0.2) (layer "B.Cu") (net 2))
 (segment (start 150.55 96.45) (end 150.8 96.2) (width 0.2) (layer "F.Cu") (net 3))
 (segment (start 151.763678 92.85) (end 152.3875 92.85) (width 0.2) (layer "F.Cu") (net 3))
 (segment (start 149.8 95.645) (end 149.8 96.42) (width 0.2) (layer "F.Cu") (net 3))
 (segment (start 150.8 96.2) (end 150.8 95.645) (width 0.2) (layer "F.Cu") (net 3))
 (segment (start 149.83 96.45) (end 150.55 96.45) (width 0.2) (layer "F.Cu") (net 3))
 (segment (start 149.8 94.794847) (end 149.8 95.645) (width 0.2) (layer "F.Cu") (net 3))
 (segment (start 149.934172 94.660675) (end 149.8 94.794847) (width 0.2) (layer "F.Cu") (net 3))
 (segment (start 149.8 96.42) (end 149.83 96.45) (width 0.2) (layer "F.Cu") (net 3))
 (segment (start 151.300869 93.312809) (end 151.763678 92.85) (width 0.2) (layer "F.Cu") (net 3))
 (via (at 149.934172 94.660675) (size 0.5) (drill 0.2) (layers "F.Cu" "B.Cu") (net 3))
 (via (at 151.300869 93.312809) (size 0.5) (drill 0.2) (layers "F.Cu" "B.Cu") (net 3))
 (segment (start 151.159921 94.843499) (end 150.116996 94.843499) (width 0.2) (layer "B.Cu") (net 3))
 (segment (start 151.6 93.61194) (end 151.6 94.40342) (width 0.2) (layer "B.Cu") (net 3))
 (segment (start 151.6 94.40342) (end 151.159921 94.843499) (width 0.2) (layer "B.Cu") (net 3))
 (segment (start 150.116996 94.843499) (end 149.934172 94.660675) (width 0.2) (layer "B.Cu") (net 3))
 (segment (start 151.300869 93.312809) (end 151.6 93.61194) (width 0.2) (layer "B.Cu") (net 3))
 (segment (start 151.397553 93.889999) (end 150.75242 93.889999) (width 0.2) (layer "F.Cu") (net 4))
 (segment (start 149.75 94.15) (end 149.3 94.6) (width 0.2) (layer "F.Cu") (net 4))
 (segment (start 150.75242 93.889999) (end 150.492419 94.15) (width 0.2) (layer "F.Cu") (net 4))
 (segment (start 150.492419 94.15) (end 149.75 94.15) (width 0.2) (layer "F.Cu") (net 4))
 (segment (start 152.3875 93.35) (end 151.937552 93.35) (width 0.2) (layer "F.Cu") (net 4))
 (segment (start 151.937552 93.35) (end 151.397553 93.889999) (width 0.2) (layer "F.Cu") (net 4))
 (segment (start 149.3 94.6) (end 149.3 95.645) (width 0.2) (layer "F.Cu") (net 4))
 (segment (start 151.85 94.843) (end 152.177 94.843) (width 0.2) (layer "F.Cu") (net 5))
 (segment (start 152.3875 93.85) (end 151.9 93.85) (width 0.2) (layer "F.Cu") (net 5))
 (segment (start 151.85 93.9) (end 151.85 94.843) (width 0.2) (layer "F.Cu") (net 5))
 (segment (start 151.9 93.85) (end 151.85 93.9) (width 0.2) (layer "F.Cu") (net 5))
 (segment (start 152.177 94.843) (end 152.3 94.966) (width 0.2) (layer "F.Cu") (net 5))
 (segment (start 152.3 94.966) (end 152.3 95.645) (width 0.2) (layer "F.Cu") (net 5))
 (segment (start 156.55 95.45) (end 157.5 94.5) (width 0.5) (layer "F.Cu") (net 6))
 (segment (start 145.25 97.35) (end 145.25 96.396) (width 0.5) (layer "F.Cu") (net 6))
 (segment (start 143.354 94.5) (end 142.35 94.5) (width 0.5) (layer "F.Cu") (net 6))
 (segment (start 157.5 94.5) (end 158.65 94.5) (width 0.5) (layer "F.Cu") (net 6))
 (segment (start 145.25 96.396) (end 143.354 94.5) (width 0.5) (layer "F.Cu") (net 6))
 (segment (start 155.3125 93.9375) (end 155.3125 93.85) (width 0.2) (layer "F.Cu") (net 6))
 (segment (start 154.5 94.75) (end 155.3125 93.9375) (width 0.2) (layer "F.Cu") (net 6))
 (via (at 156.55 95.45) (size 0.5) (drill 0.2) (layers "F.Cu" "B.Cu") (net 6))
 (via (at 154.5 94.75) (size 0.5) (drill 0.2) (layers "F.Cu" "B.Cu") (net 6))
 (via (at 145.25 97.35) (size 0.5) (drill 0.2) (layers "F.Cu" "B.Cu") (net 6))
 (segment (start 156.55 95.45) (end 155.85 94.75) (width 0.5) (layer "B.Cu") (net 6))
 (segment (start 154.079 94.75) (end 151.182 97.647) (width 0.5) (layer "B.Cu") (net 6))
 (segment (start 151.182 97.647) (end 145.547 97.647) (width 0.5) (layer "B.Cu") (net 6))
 (segment (start 155.85 94.75) (end 154.5 94.75) (width 0.5) (layer "B.Cu") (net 6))
 (segment (start 154.5 94.75) (end 154.079 94.75) (width 0.5) (layer "B.Cu") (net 6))
 (segment (start 145.547 97.647) (end 145.25 97.35) (width 0.5) (layer "B.Cu") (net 6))
 (segment (start 145.353 101.276) (end 145.854 101.777) (width 0.5) (layer "F.Cu") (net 7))
 (segment (start 156.023 97.773) (end 156.023 95.30242) (width 0.2) (layer "F.Cu") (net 7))
 (segment (start 156.75 98.5) (end 156.023 97.773) (width 0.2) (layer "F.Cu") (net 7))
 (segment (start 158.65 98.5) (end 156.75 98.5) (width 0.2) (layer "F.Cu") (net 7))
 (segment (start 156.023 95.30242) (end 156.673 94.65242) (width 0.2) (layer "F.Cu") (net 7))
 (segment (start 156.5 100.6) (end 156.5 99.646) (width 0.5) (layer "F.Cu") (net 7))
 (segment (start 142.35 98.5) (end 143.6 98.5) (width 0.5) (layer "F.Cu") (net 7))
 (segment (start 145.353 100.253) (end 145.353 101.276) (width 0.5) (layer "F.Cu") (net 7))
 (segment (start 156.2 93.35) (end 155.3125 93.35) (width 0.2) (layer "F.Cu") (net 7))
 (segment (start 157.646 98.5) (end 158.65 98.5) (width 0.5) (layer "F.Cu") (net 7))
 (segment (start 155.323 101.777) (end 156.5 100.6) (width 0.5) (layer "F.Cu") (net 7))
 (segment (start 143.6 98.5) (end 145.353 100.253) (width 0.5) (layer "F.Cu") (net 7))
 (segment (start 156.673 93.823) (end 156.2 93.35) (width 0.2) (layer "F.Cu") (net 7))
 (segment (start 156.673 94.65242) (end 156.673 93.823) (width 0.2) (layer "F.Cu") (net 7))
 (segment (start 156.5 99.646) (end 157.646 98.5) (width 0.5) (layer "F.Cu") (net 7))
 (segment (start 145.854 101.777) (end 155.323 101.777) (width 0.5) (layer "F.Cu") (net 7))
 (segment (start 146.23 96.22) (end 146.23 100.4) (width 0.5) (layer "F.Cu") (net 15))
 (segment (start 145.74 95.73) (end 146.23 96.22) (width 0.5) (layer "F.Cu") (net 15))
 (segment (start 154.87 96.22) (end 154.87 100.4) (width 0.5) (layer "F.Cu") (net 15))
 (segment (start 145.74 94.3) (end 145.74 95.73) (width 0.5) (layer "F.Cu") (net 15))
 (segment (start 154.87 100.4) (end 146.23 100.4) (width 0.5) (layer "F.Cu") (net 15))
 (segment (start 145.1 98.463994) (end 143.136006 96.5) (width 0.5) (layer "F.Cu") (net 16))
 (segment (start 157.45 96.5) (end 158.65 96.5) (width 0.5) (layer "F.Cu") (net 16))
 (segment (start 145.1 99.05) (end 145.1 98.463994) (width 0.5) (layer "F.Cu") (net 16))
 (segment (start 156.5 97.45) (end 157.45 96.5) (width 0.5) (layer "F.Cu") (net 16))
 (segment (start 143.136006 96.5) (end 142.35 96.5) (width 0.5) (layer "F.Cu") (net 16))
 (via (at 156.5 97.45) (size 0.5) (drill 0.2) (layers "F.Cu" "B.Cu") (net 16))
 (via (at 145.1 99.05) (size 0.5) (drill 0.2) (layers "F.Cu" "B.Cu") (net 16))
 (segment (start 154.95 99) (end 156.5 97.45) (width 0.5) (layer "B.Cu") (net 16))
 (segment (start 145.15 99) (end 154.95 99) (width 0.5) (layer "B.Cu") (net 16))
 (segment (start 145.1 99.05) (end 145.15 99) (width 0.5) (layer "B.Cu") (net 16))
 (segment (start 158.65 94.5) (end 157.4 94.5) (width 0.5) (layer "B.Cu") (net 19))
 (segment (start 157.4 94.5) (end 157.023 94.123) (width 0.5) (layer "B.Cu") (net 19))
 (segment (start 148.054225 95.947499) (end 146.606726 94.5) (width 0.5) (layer "B.Cu") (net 19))
 (segment (start 157.023 94.123) (end 153.441712 94.123) (width 0.5) (layer "B.Cu") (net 19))
 (segment (start 153.441712 94.123) (end 151.617213 95.947499) (width 0.5) (layer "B.Cu") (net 19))
 (segment (start 146.606726 94.5) (end 142.1 94.5) (width 0.5) (layer "B.Cu") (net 19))
 (segment (start 151.617213 95.947499) (end 148.054225 95.947499) (width 0.5) (layer "B.Cu") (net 19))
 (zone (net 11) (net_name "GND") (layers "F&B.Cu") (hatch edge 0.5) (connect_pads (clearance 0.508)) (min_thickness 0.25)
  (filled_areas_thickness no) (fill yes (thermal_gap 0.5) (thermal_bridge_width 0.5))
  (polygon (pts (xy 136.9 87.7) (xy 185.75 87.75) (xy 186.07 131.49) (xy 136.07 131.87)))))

